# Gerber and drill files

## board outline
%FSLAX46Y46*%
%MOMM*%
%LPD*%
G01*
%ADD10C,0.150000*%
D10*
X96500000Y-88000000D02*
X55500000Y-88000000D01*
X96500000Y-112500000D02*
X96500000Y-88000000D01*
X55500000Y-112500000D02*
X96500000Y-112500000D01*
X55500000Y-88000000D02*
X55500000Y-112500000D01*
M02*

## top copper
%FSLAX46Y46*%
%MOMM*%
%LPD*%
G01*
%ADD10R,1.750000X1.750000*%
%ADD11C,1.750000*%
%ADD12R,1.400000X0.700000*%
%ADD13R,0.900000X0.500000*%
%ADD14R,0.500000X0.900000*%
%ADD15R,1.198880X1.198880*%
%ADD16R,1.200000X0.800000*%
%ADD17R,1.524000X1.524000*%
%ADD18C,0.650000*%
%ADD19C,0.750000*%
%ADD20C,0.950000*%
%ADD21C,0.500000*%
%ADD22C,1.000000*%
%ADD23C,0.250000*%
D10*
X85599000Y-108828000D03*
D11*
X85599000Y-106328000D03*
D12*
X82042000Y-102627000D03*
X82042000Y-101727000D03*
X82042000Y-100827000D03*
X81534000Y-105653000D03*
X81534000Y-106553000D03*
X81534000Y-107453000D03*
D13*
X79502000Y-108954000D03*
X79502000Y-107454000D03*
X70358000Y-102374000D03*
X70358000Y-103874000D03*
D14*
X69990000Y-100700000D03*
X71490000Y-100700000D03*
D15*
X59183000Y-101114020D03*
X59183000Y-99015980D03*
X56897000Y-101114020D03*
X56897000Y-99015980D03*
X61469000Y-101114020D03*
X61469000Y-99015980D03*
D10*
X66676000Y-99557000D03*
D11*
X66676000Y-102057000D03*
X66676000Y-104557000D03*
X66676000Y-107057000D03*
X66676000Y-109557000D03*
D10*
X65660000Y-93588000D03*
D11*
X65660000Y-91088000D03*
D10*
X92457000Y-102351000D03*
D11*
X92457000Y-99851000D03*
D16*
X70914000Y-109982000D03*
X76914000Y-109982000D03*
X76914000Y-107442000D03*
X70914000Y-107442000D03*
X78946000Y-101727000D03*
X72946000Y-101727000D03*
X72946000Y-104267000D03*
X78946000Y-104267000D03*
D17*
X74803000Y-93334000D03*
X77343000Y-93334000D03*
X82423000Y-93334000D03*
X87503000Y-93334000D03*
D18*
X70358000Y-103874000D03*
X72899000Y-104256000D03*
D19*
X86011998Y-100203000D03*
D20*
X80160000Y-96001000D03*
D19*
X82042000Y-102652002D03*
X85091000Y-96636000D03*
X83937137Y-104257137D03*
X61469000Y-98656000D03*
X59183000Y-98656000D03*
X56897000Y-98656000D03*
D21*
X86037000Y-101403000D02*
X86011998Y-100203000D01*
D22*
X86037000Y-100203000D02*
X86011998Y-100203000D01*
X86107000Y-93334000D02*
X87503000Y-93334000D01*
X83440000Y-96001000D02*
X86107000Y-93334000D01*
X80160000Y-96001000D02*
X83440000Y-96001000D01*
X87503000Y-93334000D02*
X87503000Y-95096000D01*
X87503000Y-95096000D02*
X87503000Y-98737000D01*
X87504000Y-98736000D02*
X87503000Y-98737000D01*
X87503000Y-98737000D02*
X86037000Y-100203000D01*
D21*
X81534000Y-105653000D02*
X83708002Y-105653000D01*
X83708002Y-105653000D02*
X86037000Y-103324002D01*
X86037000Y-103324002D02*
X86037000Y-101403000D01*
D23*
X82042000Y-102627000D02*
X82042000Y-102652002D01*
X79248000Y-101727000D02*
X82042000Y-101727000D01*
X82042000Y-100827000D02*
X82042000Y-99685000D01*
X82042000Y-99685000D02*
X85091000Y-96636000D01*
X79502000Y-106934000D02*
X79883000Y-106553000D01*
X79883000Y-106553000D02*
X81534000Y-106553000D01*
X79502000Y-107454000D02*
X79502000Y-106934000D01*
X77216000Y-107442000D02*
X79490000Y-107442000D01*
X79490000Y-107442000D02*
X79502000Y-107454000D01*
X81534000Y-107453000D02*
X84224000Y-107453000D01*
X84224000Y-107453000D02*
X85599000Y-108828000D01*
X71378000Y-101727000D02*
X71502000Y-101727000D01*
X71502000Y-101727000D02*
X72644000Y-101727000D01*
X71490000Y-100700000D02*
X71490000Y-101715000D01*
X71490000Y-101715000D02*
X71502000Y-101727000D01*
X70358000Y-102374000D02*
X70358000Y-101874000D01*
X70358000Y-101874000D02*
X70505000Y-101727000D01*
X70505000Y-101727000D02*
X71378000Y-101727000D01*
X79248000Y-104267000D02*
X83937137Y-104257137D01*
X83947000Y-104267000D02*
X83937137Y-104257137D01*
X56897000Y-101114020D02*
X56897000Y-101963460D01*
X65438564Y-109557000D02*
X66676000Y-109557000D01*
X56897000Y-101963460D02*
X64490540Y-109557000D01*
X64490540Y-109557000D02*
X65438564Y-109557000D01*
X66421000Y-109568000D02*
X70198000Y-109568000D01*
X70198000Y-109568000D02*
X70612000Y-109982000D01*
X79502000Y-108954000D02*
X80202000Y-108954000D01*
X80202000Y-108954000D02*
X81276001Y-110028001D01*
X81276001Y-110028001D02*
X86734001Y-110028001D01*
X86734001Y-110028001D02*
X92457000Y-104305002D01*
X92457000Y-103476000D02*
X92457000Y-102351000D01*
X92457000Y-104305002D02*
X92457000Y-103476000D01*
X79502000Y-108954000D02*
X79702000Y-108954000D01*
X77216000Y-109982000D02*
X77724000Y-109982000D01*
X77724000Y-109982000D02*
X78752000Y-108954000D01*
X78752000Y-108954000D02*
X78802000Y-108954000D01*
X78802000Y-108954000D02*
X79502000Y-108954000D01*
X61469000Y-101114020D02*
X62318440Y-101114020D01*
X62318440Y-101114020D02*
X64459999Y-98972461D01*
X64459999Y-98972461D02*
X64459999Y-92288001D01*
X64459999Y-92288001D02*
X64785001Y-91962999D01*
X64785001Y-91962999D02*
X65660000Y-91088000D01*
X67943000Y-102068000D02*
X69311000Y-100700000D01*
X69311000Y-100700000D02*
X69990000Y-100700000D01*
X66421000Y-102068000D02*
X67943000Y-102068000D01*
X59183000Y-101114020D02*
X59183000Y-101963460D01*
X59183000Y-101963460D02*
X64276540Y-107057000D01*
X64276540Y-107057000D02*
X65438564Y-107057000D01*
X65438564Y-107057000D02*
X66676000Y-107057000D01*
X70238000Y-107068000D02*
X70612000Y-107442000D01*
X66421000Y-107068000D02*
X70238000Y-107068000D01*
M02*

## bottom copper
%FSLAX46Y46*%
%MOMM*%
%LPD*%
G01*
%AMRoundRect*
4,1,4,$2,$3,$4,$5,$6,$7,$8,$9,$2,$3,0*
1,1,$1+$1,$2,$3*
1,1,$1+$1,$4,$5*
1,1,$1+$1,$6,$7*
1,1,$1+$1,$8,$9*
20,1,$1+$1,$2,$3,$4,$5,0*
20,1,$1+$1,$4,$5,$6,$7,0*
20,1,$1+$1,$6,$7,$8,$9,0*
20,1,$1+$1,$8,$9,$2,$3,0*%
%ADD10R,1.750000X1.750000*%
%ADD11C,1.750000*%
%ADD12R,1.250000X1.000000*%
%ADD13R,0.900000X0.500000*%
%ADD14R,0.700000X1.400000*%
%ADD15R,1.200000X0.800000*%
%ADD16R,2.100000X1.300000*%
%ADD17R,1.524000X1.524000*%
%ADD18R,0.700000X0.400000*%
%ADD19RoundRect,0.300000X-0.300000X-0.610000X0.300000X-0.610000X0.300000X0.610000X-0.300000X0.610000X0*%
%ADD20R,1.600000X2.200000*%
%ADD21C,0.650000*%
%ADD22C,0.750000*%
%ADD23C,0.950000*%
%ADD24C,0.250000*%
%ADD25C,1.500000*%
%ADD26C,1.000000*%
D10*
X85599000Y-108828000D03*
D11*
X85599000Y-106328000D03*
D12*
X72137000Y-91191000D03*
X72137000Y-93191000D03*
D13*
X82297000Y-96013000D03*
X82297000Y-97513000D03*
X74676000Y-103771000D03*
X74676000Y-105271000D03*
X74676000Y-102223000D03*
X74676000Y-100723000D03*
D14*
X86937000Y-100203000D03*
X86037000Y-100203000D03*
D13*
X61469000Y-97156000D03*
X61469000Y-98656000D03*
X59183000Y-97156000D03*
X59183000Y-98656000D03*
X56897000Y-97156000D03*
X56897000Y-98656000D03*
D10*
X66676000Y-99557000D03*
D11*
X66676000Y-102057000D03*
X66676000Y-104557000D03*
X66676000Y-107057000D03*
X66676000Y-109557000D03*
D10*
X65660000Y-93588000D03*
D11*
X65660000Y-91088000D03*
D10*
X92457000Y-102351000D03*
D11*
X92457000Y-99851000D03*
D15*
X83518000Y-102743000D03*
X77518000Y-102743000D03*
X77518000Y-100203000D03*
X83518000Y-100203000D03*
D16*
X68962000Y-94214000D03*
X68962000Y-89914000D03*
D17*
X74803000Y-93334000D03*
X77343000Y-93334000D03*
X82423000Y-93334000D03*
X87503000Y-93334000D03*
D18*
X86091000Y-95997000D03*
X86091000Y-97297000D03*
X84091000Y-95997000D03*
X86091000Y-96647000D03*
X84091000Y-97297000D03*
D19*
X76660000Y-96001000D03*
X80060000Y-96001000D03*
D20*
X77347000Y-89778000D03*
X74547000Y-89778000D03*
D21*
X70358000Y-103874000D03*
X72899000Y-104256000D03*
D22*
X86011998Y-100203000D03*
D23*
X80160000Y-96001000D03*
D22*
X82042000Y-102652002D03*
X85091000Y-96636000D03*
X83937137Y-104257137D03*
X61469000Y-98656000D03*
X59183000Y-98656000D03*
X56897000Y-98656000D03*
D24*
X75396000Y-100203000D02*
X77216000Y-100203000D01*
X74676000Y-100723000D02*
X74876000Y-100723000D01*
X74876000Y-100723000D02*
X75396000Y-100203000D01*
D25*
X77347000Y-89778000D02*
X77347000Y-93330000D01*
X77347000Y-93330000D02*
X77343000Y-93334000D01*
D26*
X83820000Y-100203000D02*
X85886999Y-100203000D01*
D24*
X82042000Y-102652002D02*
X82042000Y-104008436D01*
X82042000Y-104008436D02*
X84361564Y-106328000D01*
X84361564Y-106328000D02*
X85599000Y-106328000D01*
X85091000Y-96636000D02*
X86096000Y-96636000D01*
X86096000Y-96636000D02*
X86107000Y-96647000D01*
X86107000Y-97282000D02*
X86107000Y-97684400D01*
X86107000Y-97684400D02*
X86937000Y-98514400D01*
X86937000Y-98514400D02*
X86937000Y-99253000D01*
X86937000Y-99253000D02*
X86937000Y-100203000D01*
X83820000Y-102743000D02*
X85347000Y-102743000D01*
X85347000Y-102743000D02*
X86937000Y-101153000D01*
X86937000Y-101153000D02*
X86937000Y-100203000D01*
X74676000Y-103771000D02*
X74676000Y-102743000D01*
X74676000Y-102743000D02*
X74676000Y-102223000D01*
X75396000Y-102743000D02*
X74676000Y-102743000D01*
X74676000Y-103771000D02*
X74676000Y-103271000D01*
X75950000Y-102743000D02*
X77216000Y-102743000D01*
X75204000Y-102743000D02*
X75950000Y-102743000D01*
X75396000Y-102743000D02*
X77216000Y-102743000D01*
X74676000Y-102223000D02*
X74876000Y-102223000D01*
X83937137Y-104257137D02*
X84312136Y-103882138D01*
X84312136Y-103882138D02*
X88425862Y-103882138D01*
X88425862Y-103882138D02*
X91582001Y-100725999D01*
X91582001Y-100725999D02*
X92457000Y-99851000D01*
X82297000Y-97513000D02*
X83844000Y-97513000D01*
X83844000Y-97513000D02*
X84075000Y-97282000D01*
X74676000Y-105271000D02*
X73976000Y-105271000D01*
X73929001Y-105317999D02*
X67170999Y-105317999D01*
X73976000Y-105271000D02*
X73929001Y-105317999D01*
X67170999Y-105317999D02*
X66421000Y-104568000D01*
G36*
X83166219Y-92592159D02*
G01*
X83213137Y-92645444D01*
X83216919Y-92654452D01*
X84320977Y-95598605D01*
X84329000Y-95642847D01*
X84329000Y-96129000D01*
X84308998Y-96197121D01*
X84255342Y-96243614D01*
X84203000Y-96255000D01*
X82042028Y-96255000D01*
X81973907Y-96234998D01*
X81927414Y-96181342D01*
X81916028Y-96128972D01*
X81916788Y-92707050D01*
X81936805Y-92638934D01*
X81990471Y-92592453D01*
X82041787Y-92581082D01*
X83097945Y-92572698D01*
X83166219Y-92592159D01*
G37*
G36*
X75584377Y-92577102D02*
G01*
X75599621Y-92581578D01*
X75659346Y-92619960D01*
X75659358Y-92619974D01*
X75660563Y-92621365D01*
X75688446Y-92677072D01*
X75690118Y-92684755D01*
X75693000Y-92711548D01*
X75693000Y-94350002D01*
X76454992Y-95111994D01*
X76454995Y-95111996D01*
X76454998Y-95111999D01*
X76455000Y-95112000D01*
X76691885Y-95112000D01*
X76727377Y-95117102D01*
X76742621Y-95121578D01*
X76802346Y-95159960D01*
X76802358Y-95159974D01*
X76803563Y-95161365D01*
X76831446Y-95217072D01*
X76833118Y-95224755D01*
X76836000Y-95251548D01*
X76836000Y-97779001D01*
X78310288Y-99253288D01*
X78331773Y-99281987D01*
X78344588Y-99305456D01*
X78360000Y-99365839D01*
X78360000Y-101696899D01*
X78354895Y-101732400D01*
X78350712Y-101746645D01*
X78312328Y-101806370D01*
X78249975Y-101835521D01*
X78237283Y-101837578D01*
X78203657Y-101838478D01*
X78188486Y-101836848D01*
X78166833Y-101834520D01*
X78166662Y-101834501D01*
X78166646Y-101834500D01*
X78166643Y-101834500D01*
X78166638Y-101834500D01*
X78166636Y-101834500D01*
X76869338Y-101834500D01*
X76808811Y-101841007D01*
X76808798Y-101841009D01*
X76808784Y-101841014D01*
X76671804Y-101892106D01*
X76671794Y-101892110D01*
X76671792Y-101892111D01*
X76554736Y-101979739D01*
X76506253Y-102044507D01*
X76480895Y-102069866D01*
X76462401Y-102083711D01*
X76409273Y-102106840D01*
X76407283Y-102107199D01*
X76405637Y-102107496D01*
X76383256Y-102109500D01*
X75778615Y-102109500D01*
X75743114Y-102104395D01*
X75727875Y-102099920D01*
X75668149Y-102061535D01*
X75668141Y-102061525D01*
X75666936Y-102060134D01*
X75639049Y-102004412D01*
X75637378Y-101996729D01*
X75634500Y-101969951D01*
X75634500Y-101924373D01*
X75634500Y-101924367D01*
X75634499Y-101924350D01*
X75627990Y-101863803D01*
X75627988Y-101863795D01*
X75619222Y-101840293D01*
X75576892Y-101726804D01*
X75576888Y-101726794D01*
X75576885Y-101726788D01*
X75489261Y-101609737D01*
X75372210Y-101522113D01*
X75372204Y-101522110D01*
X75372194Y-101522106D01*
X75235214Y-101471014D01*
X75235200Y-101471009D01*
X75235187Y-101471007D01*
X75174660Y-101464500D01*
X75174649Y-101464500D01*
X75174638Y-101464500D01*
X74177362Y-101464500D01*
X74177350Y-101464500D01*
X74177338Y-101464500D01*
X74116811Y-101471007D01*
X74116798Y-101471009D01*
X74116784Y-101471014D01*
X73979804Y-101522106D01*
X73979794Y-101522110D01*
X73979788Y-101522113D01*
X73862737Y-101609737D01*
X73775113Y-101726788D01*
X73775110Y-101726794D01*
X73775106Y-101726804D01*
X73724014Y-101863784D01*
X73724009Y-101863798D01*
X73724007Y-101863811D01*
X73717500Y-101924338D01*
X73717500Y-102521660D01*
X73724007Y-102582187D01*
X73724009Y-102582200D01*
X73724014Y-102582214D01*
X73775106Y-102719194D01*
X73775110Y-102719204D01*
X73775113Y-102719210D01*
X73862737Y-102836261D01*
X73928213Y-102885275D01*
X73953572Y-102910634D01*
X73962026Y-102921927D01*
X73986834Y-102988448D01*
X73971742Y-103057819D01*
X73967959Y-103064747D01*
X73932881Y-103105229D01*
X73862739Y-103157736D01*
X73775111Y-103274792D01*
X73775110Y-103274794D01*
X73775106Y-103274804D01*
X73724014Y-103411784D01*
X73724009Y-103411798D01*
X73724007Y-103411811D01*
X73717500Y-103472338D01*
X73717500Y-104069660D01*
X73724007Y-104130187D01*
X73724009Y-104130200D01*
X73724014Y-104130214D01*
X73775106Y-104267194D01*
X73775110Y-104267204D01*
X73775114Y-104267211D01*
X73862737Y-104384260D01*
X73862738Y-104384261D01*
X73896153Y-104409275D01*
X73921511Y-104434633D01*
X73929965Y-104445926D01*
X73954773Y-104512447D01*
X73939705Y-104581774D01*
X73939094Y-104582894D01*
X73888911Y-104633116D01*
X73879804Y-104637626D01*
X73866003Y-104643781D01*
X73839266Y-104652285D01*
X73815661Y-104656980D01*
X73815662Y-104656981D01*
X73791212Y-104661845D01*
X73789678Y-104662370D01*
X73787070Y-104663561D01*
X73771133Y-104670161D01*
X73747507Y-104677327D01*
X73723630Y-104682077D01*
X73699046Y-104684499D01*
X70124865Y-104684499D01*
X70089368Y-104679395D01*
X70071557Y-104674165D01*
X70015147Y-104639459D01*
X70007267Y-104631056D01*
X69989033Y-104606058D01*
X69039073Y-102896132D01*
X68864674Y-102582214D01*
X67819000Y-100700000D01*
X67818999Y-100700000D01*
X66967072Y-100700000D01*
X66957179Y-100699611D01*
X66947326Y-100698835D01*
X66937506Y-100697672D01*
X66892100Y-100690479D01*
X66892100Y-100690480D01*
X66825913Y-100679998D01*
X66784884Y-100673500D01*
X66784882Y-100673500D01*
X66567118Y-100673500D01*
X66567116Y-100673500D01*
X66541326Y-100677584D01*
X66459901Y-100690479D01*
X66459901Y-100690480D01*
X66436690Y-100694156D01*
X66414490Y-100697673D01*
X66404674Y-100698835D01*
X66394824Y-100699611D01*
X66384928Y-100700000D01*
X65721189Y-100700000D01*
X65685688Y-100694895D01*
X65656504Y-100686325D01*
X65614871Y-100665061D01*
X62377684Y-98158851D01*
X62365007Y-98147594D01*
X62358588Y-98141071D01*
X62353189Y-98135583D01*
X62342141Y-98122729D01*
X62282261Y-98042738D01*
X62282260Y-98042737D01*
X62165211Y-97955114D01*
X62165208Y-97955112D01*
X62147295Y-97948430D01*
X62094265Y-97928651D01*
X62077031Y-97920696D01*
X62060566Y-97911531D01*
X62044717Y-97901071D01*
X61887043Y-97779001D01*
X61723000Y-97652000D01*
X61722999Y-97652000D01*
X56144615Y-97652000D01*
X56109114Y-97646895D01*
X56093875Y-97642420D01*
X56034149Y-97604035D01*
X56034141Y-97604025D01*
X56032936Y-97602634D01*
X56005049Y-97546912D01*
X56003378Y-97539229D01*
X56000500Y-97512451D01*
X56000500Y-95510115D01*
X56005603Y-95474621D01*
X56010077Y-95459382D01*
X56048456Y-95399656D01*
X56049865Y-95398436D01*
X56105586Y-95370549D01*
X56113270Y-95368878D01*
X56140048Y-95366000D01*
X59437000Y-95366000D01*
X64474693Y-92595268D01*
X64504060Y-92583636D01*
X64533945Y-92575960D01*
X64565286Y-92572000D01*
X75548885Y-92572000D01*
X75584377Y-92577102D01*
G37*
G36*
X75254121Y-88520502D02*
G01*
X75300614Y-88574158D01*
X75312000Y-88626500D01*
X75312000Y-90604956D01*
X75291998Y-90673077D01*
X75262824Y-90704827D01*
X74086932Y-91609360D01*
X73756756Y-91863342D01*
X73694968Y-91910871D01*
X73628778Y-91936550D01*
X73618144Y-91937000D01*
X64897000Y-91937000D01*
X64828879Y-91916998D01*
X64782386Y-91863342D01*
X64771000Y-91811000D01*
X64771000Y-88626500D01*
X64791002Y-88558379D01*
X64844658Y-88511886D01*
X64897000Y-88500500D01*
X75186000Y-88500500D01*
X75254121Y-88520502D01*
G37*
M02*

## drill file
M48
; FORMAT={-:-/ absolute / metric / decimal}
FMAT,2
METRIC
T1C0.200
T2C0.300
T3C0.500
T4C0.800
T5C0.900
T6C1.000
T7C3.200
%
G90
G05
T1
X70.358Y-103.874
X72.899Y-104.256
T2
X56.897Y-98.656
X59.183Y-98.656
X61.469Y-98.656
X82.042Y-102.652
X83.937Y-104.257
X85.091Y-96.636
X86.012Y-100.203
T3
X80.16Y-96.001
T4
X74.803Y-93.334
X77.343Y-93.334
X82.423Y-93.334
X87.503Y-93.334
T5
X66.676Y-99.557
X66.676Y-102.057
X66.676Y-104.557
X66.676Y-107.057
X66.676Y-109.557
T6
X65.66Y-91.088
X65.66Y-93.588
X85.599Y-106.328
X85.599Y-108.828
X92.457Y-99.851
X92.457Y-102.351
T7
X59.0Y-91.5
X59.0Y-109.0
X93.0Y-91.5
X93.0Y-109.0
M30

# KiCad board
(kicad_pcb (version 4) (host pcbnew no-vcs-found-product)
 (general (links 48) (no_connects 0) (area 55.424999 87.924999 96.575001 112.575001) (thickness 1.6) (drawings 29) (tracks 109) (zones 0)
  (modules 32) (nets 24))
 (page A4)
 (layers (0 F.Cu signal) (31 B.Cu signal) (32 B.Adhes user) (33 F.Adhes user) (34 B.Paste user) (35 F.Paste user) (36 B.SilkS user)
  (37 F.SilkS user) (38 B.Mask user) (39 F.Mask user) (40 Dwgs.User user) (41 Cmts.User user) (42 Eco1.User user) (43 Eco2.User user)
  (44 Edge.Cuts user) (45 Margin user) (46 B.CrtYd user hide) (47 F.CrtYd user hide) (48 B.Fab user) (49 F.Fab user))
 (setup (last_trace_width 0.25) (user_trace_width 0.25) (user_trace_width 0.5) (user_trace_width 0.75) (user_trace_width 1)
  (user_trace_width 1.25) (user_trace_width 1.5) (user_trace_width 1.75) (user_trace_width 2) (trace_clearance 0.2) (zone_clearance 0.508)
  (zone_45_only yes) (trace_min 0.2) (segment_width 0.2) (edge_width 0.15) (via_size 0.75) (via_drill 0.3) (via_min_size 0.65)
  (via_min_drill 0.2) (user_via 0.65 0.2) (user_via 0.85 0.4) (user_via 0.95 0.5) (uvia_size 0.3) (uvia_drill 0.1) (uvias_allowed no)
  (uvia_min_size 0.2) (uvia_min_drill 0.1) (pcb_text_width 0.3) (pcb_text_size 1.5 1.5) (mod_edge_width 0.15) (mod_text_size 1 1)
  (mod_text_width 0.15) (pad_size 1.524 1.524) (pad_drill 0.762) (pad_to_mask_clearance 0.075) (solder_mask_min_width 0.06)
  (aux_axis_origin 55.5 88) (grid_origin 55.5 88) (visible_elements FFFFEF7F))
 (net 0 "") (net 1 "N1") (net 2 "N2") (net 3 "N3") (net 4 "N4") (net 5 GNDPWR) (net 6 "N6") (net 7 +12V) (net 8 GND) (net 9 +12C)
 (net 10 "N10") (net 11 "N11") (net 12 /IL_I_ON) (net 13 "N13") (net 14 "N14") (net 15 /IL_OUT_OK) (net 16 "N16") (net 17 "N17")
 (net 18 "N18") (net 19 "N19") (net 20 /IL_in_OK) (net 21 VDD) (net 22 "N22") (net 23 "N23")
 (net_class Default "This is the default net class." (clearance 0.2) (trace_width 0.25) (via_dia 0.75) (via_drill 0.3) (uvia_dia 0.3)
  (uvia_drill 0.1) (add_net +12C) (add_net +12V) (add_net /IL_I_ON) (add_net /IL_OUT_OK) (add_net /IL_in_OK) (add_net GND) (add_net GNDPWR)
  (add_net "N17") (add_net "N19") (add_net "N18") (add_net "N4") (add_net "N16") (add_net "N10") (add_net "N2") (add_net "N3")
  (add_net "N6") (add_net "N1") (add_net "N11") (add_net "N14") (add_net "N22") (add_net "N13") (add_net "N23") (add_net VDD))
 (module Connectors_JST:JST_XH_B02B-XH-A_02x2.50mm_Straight (layer F.Cu) (at 85.599 108.828 90)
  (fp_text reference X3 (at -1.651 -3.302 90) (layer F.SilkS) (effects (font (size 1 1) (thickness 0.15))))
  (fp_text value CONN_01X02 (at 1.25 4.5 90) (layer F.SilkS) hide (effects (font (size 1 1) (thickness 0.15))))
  (pad 1 thru_hole rect (at 0 0 90) (size 1.75 1.75) (drill 1) (layers *.Cu *.Mask) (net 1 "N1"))
  (pad 2 thru_hole circle (at 2.5 0 90) (size 1.75 1.75) (drill 1) (layers *.Cu *.Mask) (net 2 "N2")))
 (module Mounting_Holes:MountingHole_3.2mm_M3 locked (layer F.Cu) (at 93 109)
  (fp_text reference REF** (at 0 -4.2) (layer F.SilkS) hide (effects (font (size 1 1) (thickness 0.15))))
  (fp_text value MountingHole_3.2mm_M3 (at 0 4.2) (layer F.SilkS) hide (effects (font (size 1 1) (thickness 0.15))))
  (pad 1 np_thru_hole circle (at 0 0) (size 3.2 3.2) (drill 3.2) (layers *.Cu *.Mask F.SilkS)))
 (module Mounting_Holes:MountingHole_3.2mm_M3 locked (layer F.Cu) (at 59 91.5)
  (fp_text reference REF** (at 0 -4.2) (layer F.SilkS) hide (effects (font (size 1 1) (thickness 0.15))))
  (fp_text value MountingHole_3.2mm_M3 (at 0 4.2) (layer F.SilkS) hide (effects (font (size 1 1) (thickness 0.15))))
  (pad 1 np_thru_hole circle (at 0 0) (size 3.2 3.2) (drill 3.2) (layers *.Cu *.Mask F.SilkS)))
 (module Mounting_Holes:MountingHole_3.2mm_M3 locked (layer F.Cu) (at 59 109)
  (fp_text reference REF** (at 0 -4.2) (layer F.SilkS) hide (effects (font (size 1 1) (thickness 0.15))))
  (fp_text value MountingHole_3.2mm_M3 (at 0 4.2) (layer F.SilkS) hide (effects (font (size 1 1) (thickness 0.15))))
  (pad 1 np_thru_hole circle (at 0 0) (size 3.2 3.2) (drill 3.2) (layers *.Cu *.Mask F.SilkS)))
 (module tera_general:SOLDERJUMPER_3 (layer F.Cu) (at 82.042 101.727 180)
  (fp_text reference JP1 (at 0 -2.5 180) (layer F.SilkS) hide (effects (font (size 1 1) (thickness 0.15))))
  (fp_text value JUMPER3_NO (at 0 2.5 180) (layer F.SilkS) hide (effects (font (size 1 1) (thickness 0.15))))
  (pad 1 smd rect (at 0 -0.9 180) (size 1.4 0.7) (layers F.Cu F.Paste F.Mask) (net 2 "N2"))
  (pad 2 smd rect (at 0 0 180) (size 1.4 0.7) (layers F.Cu F.Paste F.Mask) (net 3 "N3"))
  (pad 3 smd rect (at 0 0.9 180) (size 1.4 0.7) (layers F.Cu F.Paste F.Mask) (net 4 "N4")))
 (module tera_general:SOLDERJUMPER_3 (layer F.Cu) (at 81.534 106.553)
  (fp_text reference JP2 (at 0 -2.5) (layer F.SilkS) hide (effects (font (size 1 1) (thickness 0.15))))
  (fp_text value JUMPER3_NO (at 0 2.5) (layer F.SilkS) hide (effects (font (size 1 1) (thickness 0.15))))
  (pad 1 smd rect (at 0 -0.9) (size 1.4 0.7) (layers F.Cu F.Paste F.Mask) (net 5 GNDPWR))
  (pad 2 smd rect (at 0 0) (size 1.4 0.7) (layers F.Cu F.Paste F.Mask) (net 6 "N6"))
  (pad 3 smd rect (at 0 0.9) (size 1.4 0.7) (layers F.Cu F.Paste F.Mask) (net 1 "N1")))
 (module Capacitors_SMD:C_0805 (layer B.Cu) (at 72.137 92.191 270)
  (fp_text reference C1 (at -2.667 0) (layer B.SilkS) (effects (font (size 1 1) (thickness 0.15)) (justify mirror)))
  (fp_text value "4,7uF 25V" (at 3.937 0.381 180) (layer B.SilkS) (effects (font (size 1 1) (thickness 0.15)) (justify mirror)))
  (pad 1 smd rect (at -1 0 270) (size 1 1.25) (layers B.Cu B.Paste B.Mask) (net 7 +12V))
  (pad 2 smd rect (at 1 0 270) (size 1 1.25) (layers B.Cu B.Paste B.Mask) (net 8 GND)))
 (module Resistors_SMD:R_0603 (layer B.Cu) (at 82.297 96.763 270)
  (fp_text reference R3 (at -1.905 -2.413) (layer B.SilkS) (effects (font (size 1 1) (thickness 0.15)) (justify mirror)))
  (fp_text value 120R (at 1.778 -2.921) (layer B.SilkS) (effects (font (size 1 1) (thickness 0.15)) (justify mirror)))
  (pad 1 smd rect (at -0.75 0 270) (size 0.5 0.9) (layers B.Cu B.Paste B.Mask) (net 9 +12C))
  (pad 2 smd rect (at 0.75 0 270) (size 0.5 0.9) (layers B.Cu B.Paste B.Mask) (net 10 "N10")))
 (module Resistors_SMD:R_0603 (layer B.Cu) (at 74.676 104.521 270)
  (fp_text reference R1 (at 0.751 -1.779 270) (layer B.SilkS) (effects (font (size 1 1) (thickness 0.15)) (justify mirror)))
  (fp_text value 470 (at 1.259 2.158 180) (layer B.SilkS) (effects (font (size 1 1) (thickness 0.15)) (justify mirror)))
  (pad 1 smd rect (at -0.75 0 270) (size 0.5 0.9) (layers B.Cu B.Paste B.Mask) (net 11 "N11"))
  (pad 2 smd rect (at 0.75 0 270) (size 0.5 0.9) (layers B.Cu B.Paste B.Mask) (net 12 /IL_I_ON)))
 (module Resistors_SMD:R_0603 (layer B.Cu) (at 74.676 101.473 90)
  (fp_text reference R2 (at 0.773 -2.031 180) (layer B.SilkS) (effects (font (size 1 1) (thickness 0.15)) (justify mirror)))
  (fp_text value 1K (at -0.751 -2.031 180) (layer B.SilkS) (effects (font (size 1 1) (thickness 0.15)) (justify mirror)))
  (pad 1 smd rect (at -0.75 0 90) (size 0.5 0.9) (layers B.Cu B.Paste B.Mask) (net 11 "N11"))
  (pad 2 smd rect (at 0.75 0 90) (size 0.5 0.9) (layers B.Cu B.Paste B.Mask) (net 8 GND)))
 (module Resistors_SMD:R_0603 (layer F.Cu) (at 79.502 108.204 90)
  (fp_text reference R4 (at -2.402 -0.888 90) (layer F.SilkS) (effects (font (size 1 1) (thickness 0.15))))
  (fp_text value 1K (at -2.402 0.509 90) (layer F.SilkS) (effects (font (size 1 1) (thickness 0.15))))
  (pad 1 smd rect (at -0.75 0 90) (size 0.5 0.9) (layers F.Cu F.Paste F.Mask) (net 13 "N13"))
  (pad 2 smd rect (at 0.75 0 90) (size 0.5 0.9) (layers F.Cu F.Paste F.Mask) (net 6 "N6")))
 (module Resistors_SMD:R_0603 (layer F.Cu) (at 70.358 103.124 270)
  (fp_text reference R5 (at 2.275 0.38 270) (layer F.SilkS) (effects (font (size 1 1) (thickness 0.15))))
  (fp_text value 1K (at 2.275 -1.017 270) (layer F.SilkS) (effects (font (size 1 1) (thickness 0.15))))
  (pad 1 smd rect (at -0.75 0 270) (size 0.5 0.9) (layers F.Cu F.Paste F.Mask) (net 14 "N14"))
  (pad 2 smd rect (at 0.75 0 270) (size 0.5 0.9) (layers F.Cu F.Paste F.Mask) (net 8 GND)))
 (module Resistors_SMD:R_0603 (layer F.Cu) (at 70.74 100.7)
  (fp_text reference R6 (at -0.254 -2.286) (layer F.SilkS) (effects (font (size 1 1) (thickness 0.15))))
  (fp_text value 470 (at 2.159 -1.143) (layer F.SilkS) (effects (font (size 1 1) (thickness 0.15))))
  (pad 1 smd rect (at -0.75 0) (size 0.5 0.9) (layers F.Cu F.Paste F.Mask) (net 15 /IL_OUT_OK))
  (pad 2 smd rect (at 0.75 0) (size 0.5 0.9) (layers F.Cu F.Paste F.Mask) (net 14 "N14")))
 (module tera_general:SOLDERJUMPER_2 (layer B.Cu) (at 86.487 100.203 90)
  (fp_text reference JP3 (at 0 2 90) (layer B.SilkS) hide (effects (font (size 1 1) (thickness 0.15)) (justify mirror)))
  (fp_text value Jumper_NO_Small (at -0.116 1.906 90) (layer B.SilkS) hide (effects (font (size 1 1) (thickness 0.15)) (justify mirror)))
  (pad 1 smd rect (at 0 0.45 90) (size 1.4 0.7) (layers B.Cu B.Paste B.Mask) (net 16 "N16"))
  (pad 2 smd rect (at 0 -0.45 90) (size 1.4 0.7) (layers B.Cu B.Paste B.Mask) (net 5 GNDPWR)))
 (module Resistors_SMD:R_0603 (layer B.Cu) (at 61.469 97.906 270)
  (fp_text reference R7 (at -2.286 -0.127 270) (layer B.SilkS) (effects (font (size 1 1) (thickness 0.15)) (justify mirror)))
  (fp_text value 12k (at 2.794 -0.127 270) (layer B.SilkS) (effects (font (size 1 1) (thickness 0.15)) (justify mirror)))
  (pad 1 smd rect (at -0.75 0 270) (size 0.5 0.9) (layers B.Cu B.Paste B.Mask) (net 8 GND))
  (pad 2 smd rect (at 0.75 0 270) (size 0.5 0.9) (layers B.Cu B.Paste B.Mask) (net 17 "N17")))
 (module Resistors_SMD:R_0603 (layer B.Cu) (at 59.183 97.906 270)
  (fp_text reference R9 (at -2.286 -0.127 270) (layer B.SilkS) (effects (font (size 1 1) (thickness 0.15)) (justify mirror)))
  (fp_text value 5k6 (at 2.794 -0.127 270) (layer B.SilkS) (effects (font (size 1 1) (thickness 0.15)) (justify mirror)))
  (pad 1 smd rect (at -0.75 0 270) (size 0.5 0.9) (layers B.Cu B.Paste B.Mask) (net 8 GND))
  (pad 2 smd rect (at 0.75 0 270) (size 0.5 0.9) (layers B.Cu B.Paste B.Mask) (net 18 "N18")))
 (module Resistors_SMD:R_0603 (layer B.Cu) (at 56.897 97.906 270)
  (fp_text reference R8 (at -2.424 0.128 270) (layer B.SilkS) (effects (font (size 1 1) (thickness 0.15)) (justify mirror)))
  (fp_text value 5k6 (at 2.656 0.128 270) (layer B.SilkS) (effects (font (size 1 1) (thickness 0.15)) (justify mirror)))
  (pad 1 smd rect (at -0.75 0 270) (size 0.5 0.9) (layers B.Cu B.Paste B.Mask) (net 8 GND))
  (pad 2 smd rect (at 0.75 0 270) (size 0.5 0.9) (layers B.Cu B.Paste B.Mask) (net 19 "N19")))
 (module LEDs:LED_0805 (layer F.Cu) (at 59.183 100.065 270)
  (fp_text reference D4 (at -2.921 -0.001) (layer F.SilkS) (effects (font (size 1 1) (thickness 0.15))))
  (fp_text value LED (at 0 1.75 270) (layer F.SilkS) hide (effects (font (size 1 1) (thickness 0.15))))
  (pad 2 smd rect (at 1.04902 0 90) (size 1.19888 1.19888) (layers F.Cu F.Paste F.Mask) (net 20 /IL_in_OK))
  (pad 1 smd rect (at -1.04902 0 90) (size 1.19888 1.19888) (layers F.Cu F.Paste F.Mask) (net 18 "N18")))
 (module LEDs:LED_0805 (layer F.Cu) (at 56.897 100.065 270)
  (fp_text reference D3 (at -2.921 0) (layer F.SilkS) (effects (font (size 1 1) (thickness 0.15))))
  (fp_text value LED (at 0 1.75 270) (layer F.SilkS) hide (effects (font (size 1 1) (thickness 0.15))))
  (pad 2 smd rect (at 1.04902 0 90) (size 1.19888 1.19888) (layers F.Cu F.Paste F.Mask) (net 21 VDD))
  (pad 1 smd rect (at -1.04902 0 90) (size 1.19888 1.19888) (layers F.Cu F.Paste F.Mask) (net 19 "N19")))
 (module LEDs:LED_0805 (layer F.Cu) (at 61.469 100.065 270)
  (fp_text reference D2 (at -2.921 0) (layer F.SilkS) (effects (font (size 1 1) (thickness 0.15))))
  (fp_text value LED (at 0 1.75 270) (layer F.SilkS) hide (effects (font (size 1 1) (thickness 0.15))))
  (pad 2 smd rect (at 1.04902 0 90) (size 1.19888 1.19888) (layers F.Cu F.Paste F.Mask) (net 7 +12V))
  (pad 1 smd rect (at -1.04902 0 90) (size 1.19888 1.19888) (layers F.Cu F.Paste F.Mask) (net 17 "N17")))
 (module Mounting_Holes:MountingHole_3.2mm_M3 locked (layer F.Cu) (at 93 91.5)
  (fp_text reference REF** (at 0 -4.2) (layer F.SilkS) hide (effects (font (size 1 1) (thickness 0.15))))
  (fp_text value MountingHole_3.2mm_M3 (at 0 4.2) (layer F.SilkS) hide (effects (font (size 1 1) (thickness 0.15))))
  (pad 1 np_thru_hole circle (at 0 0) (size 3.2 3.2) (drill 3.2) (layers *.Cu *.Mask F.SilkS)))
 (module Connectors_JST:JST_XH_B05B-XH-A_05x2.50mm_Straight (layer F.Cu) (at 66.676 99.557 270)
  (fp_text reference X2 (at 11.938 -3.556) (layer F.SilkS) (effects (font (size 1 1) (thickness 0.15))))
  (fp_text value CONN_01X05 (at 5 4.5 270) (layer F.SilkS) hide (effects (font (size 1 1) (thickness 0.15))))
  (pad 1 thru_hole rect (at 0 0 270) (size 1.75 1.75) (drill 0.9) (layers *.Cu *.Mask) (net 8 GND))
  (pad 2 thru_hole circle (at 2.5 0 270) (size 1.75 1.75) (drill 0.9) (layers *.Cu *.Mask) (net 15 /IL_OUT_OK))
  (pad 3 thru_hole circle (at 5 0 270) (size 1.75 1.75) (drill 0.9) (layers *.Cu *.Mask) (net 12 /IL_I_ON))
  (pad 4 thru_hole circle (at 7.5 0 270) (size 1.75 1.75) (drill 0.9) (layers *.Cu *.Mask) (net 20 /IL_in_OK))
  (pad 5 thru_hole circle (at 10 0 270) (size 1.75 1.75) (drill 0.9) (layers *.Cu *.Mask) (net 21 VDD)))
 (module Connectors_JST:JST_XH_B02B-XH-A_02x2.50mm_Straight (layer F.Cu) (at 65.66 93.588 90)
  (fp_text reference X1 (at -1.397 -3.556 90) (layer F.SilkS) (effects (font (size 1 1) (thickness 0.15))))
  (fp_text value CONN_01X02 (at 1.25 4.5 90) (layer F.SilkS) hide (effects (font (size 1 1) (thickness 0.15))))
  (pad 1 thru_hole rect (at 0 0 90) (size 1.75 1.75) (drill 1) (layers *.Cu *.Mask) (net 8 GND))
  (pad 2 thru_hole circle (at 2.5 0 90) (size 1.75 1.75) (drill 1) (layers *.Cu *.Mask) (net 7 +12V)))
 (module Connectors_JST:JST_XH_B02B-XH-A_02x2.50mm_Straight (layer F.Cu) (at 92.457 102.351 90)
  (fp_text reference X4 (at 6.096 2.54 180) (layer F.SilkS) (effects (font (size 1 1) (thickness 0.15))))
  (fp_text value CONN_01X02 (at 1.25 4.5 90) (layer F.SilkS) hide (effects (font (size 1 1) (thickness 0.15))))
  (pad 1 thru_hole rect (at 0 0 90) (size 1.75 1.75) (drill 1) (layers *.Cu *.Mask) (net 13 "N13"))
  (pad 2 thru_hole circle (at 2.5 0 90) (size 1.75 1.75) (drill 1) (layers *.Cu *.Mask) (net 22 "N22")))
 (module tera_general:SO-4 (layer B.Cu) (at 80.518 101.473 90)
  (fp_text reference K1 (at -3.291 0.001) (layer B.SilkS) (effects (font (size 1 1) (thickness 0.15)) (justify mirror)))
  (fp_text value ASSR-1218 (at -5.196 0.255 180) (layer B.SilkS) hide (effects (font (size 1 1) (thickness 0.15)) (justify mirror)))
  (pad 4 smd rect (at -1.27 3 90) (size 0.8 1.2) (layers B.Cu B.Paste B.Mask) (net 16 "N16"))
  (pad 1 smd rect (at -1.27 -3 90) (size 0.8 1.2) (layers B.Cu B.Paste B.Mask) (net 11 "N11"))
  (pad 2 smd rect (at 1.27 -3 90) (size 0.8 1.2) (layers B.Cu B.Paste B.Mask) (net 8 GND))
  (pad 3 smd rect (at 1.27 3 90) (size 0.8 1.2) (layers B.Cu B.Paste B.Mask) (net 5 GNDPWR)))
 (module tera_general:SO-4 (layer F.Cu) (at 73.914 108.712 90)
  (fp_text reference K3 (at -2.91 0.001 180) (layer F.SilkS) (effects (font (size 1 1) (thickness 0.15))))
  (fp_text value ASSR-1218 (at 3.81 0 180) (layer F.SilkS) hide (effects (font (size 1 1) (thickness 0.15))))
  (pad 4 smd rect (at -1.27 -3 90) (size 0.8 1.2) (layers F.Cu F.Paste F.Mask) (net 21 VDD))
  (pad 1 smd rect (at -1.27 3 90) (size 0.8 1.2) (layers F.Cu F.Paste F.Mask) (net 13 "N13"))
  (pad 2 smd rect (at 1.27 3 90) (size 0.8 1.2) (layers F.Cu F.Paste F.Mask) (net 6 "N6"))
  (pad 3 smd rect (at 1.27 -3 90) (size 0.8 1.2) (layers F.Cu F.Paste F.Mask) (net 20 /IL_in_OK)))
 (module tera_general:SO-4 (layer F.Cu) (at 75.946 102.997 270)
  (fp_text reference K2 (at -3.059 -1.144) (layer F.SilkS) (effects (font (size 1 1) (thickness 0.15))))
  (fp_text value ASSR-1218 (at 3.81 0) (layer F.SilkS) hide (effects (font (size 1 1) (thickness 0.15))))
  (pad 4 smd rect (at -1.27 -3 270) (size 0.8 1.2) (layers F.Cu F.Paste F.Mask) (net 3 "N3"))
  (pad 1 smd rect (at -1.27 3 270) (size 0.8 1.2) (layers F.Cu F.Paste F.Mask) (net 14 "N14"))
  (pad 2 smd rect (at 1.27 3 270) (size 0.8 1.2) (layers F.Cu F.Paste F.Mask) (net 8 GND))
  (pad 3 smd rect (at 1.27 -3 270) (size 0.8 1.2) (layers F.Cu F.Paste F.Mask) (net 22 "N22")))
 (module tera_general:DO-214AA (layer B.Cu) (at 68.962 92.064 270)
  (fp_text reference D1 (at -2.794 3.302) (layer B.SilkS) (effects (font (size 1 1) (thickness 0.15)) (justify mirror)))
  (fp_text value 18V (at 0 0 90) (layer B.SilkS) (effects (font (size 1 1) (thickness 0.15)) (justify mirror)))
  (pad 2 smd rect (at 2.15 0 270) (size 1.3 2.1) (layers B.Cu B.Paste B.Mask) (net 8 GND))
  (pad 1 smd rect (at -2.15 0 270) (size 1.3 2.1) (layers B.Cu B.Paste B.Mask) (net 7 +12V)))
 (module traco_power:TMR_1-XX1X (layer F.Cu) (at 74.803 93.334)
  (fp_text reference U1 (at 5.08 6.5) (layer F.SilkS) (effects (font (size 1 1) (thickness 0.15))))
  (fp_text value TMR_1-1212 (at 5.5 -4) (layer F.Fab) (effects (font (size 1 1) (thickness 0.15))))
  (pad 1 thru_hole rect (at 0 0) (size 1.524 1.524) (drill 0.8) (layers *.Cu *.Mask) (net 8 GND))
  (pad 2 thru_hole rect (at 2.54 0) (size 1.524 1.524) (drill 0.8) (layers *.Cu *.Mask) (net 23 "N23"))
  (pad 4 thru_hole rect (at 7.62 0) (size 1.524 1.524) (drill 0.8) (layers *.Cu *.Mask) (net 9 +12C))
  (pad 6 thru_hole rect (at 12.7 0) (size 1.524 1.524) (drill 0.8) (layers *.Cu *.Mask) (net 5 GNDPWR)))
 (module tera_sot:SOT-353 (layer B.Cu) (at 85.091 96.647 180)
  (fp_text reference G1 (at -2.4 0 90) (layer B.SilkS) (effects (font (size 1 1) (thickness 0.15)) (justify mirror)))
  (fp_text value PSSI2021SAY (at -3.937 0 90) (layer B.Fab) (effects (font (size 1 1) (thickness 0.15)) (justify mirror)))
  (pad 1 smd rect (at -1 0.65 180) (size 0.7 0.4) (layers B.Cu B.Paste B.Mask))
  (pad 3 smd rect (at -1 -0.65 180) (size 0.7 0.4) (layers B.Cu B.Paste B.Mask) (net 16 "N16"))
  (pad 5 smd rect (at 1 0.65 180) (size 0.7 0.4) (layers B.Cu B.Paste B.Mask) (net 9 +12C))
  (pad 2 smd rect (at -1 0 180) (size 0.7 0.4) (layers B.Cu B.Paste B.Mask) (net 4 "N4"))
  (pad 4 smd rect (at 1 -0.65 180) (size 0.7 0.4) (layers B.Cu B.Paste B.Mask) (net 10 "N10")))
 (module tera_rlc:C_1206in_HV (layer B.Cu) (at 78.36 96.001)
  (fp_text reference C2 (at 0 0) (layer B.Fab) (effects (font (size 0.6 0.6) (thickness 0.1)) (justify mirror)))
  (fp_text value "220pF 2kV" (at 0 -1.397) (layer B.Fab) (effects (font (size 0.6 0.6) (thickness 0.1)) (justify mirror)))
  (pad 1 smd roundrect (at -1.7 0) (size 1.2 1.82) (layers B.Cu B.Paste B.Mask) (roundrect_rratio 0.25) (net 8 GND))
  (pad 2 smd roundrect (at 1.7 0) (size 1.2 1.82) (layers B.Cu B.Paste B.Mask) (roundrect_rratio 0.25) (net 5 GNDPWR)))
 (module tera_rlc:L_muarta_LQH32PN (layer B.Cu) (at 75.947 89.778 180)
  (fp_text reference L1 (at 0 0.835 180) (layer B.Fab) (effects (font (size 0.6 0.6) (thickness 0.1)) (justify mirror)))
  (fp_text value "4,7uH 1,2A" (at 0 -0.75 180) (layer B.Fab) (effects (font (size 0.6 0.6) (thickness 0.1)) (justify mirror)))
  (pad 1 smd rect (at -1.4 0 180) (size 1.6 2.2) (layers B.Cu B.Paste B.Mask) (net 23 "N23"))
  (pad 2 smd rect (at 1.4 0 180) (size 1.6 2.2) (layers B.Cu B.Paste B.Mask) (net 7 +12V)))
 (gr_line (start 96.5 88) (end 55.5 88) (layer Edge.Cuts) (width 0.15))
 (gr_line (start 96.5 112.5) (end 96.5 88) (layer Edge.Cuts) (width 0.15))
 (gr_line (start 55.5 112.5) (end 96.5 112.5) (layer Edge.Cuts) (width 0.15))
 (gr_line (start 55.5 88) (end 55.5 112.5) (layer Edge.Cuts) (width 0.15))
 (via (at 70.358 103.874) (size 0.65) (drill 0.2) (layers F.Cu B.Cu) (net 8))
 (via (at 72.899 104.256) (size 0.65) (drill 0.2) (layers F.Cu B.Cu) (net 8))
 (segment (start 75.396 100.203) (end 77.216 100.203) (width 0.25) (layer B.Cu) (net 8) (status 20))
 (segment (start 74.676 100.723) (end 74.876 100.723) (width 0.25) (layer B.Cu) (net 8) (status 30))
 (segment (start 74.876 100.723) (end 75.396 100.203) (width 0.25) (layer B.Cu) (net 8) (status 10))
 (segment (start 77.347 89.778) (end 77.347 93.33) (width 1.5) (layer B.Cu) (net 23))
 (segment (start 77.347 93.33) (end 77.343 93.334) (width 1.5) (layer B.Cu) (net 23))
 (segment (start 86.037 101.403) (end 86.011998 100.203) (width 0.5) (layer F.Cu) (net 5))
 (segment (start 86.037 100.203) (end 86.011998 100.203) (width 1) (layer F.Cu) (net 5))
 (via (at 86.011998 100.203) (size 0.75) (drill 0.3) (layers F.Cu B.Cu) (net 5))
 (segment (start 86.107 93.334) (end 87.503 93.334) (width 1) (layer F.Cu) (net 5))
 (segment (start 83.44 96.001) (end 86.107 93.334) (width 1) (layer F.Cu) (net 5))
 (segment (start 80.16 96.001) (end 83.44 96.001) (width 1) (layer F.Cu) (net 5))
 (via (at 80.16 96.001) (size 0.95) (drill 0.5) (layers F.Cu B.Cu) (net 5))
 (segment (start 87.503 93.334) (end 87.503 95.096) (width 1) (layer F.Cu) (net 5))
 (segment (start 87.503 95.096) (end 87.503 98.737) (width 1) (layer F.Cu) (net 5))
 (segment (start 87.504 98.736) (end 87.503 98.737) (width 1) (layer F.Cu) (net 5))
 (segment (start 87.503 98.737) (end 86.037 100.203) (width 1) (layer F.Cu) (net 5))
 (segment (start 81.534 105.653) (end 83.708002 105.653) (width 0.5) (layer F.Cu) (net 5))
 (segment (start 83.708002 105.653) (end 86.037 103.324002) (width 0.5) (layer F.Cu) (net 5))
 (segment (start 86.037 103.324002) (end 86.037 101.403) (width 0.5) (layer F.Cu) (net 5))
 (segment (start 83.82 100.203) (end 85.886999 100.203) (width 1) (layer B.Cu) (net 5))
 (segment (start 82.042 102.652002) (end 82.042 104.008436) (width 0.25) (layer B.Cu) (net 2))
 (segment (start 82.042 104.008436) (end 84.361564 106.328) (width 0.25) (layer B.Cu) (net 2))
 (segment (start 84.361564 106.328) (end 85.599 106.328) (width 0.25) (layer B.Cu) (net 2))
 (segment (start 82.042 102.627) (end 82.042 102.652002) (width 0.25) (layer F.Cu) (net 2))
 (via (at 82.042 102.652002) (size 0.75) (drill 0.3) (layers F.Cu B.Cu) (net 2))
 (segment (start 79.248 101.727) (end 82.042 101.727) (width 0.25) (layer F.Cu) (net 3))
 (segment (start 85.091 96.636) (end 86.096 96.636) (width 0.25) (layer B.Cu) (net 4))
 (segment (start 86.096 96.636) (end 86.107 96.647) (width 0.25) (layer B.Cu) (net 4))
 (segment (start 82.042 100.827) (end 82.042 99.685) (width 0.25) (layer F.Cu) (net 4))
 (segment (start 82.042 99.685) (end 85.091 96.636) (width 0.25) (layer F.Cu) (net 4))
 (via (at 85.091 96.636) (size 0.75) (drill 0.3) (layers F.Cu B.Cu) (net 4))
 (segment (start 79.502 106.934) (end 79.883 106.553) (width 0.25) (layer F.Cu) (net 6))
 (segment (start 79.883 106.553) (end 81.534 106.553) (width 0.25) (layer F.Cu) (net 6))
 (segment (start 79.502 107.454) (end 79.502 106.934) (width 0.25) (layer F.Cu) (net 6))
 (segment (start 77.216 107.442) (end 79.49 107.442) (width 0.25) (layer F.Cu) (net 6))
 (segment (start 79.49 107.442) (end 79.502 107.454) (width 0.25) (layer F.Cu) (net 6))
 (segment (start 81.534 107.453) (end 84.224 107.453) (width 0.25) (layer F.Cu) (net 1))
 (segment (start 84.224 107.453) (end 85.599 108.828) (width 0.25) (layer F.Cu) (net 1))
 (segment (start 86.107 97.282) (end 86.107 97.6844) (width 0.25) (layer B.Cu) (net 16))
 (segment (start 86.107 97.6844) (end 86.937 98.5144) (width 0.25) (layer B.Cu) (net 16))
 (segment (start 86.937 98.5144) (end 86.937 99.253) (width 0.25) (layer B.Cu) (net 16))
 (segment (start 86.937 99.253) (end 86.937 100.203) (width 0.25) (layer B.Cu) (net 16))
 (segment (start 83.82 102.743) (end 85.347 102.743) (width 0.25) (layer B.Cu) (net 16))
 (segment (start 85.347 102.743) (end 86.937 101.153) (width 0.25) (layer B.Cu) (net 16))
 (segment (start 86.937 101.153) (end 86.937 100.203) (width 0.25) (layer B.Cu) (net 16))
 (segment (start 74.676 103.771) (end 74.676 102.743) (width 0.25) (layer B.Cu) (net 11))
 (segment (start 74.676 102.743) (end 74.676 102.223) (width 0.25) (layer B.Cu) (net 11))
 (segment (start 75.396 102.743) (end 74.676 102.743) (width 0.25) (layer B.Cu) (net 11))
 (segment (start 74.676 103.771) (end 74.676 103.271) (width 0.25) (layer B.Cu) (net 11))
 (segment (start 75.95 102.743) (end 77.216 102.743) (width 0.25) (layer B.Cu) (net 11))
 (segment (start 75.204 102.743) (end 75.95 102.743) (width 0.25) (layer B.Cu) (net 11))
 (segment (start 75.396 102.743) (end 77.216 102.743) (width 0.25) (layer B.Cu) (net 11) (status 20))
 (segment (start 74.676 102.223) (end 74.876 102.223) (width 0.25) (layer B.Cu) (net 11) (status 30))
 (segment (start 71.378 101.727) (end 71.502 101.727) (width 0.25) (layer F.Cu) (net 14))
 (segment (start 71.502 101.727) (end 72.644 101.727) (width 0.25) (layer F.Cu) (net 14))
 (segment (start 71.49 100.7) (end 71.49 101.715) (width 0.25) (layer F.Cu) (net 14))
 (segment (start 71.49 101.715) (end 71.502 101.727) (width 0.25) (layer F.Cu) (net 14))
 (segment (start 70.358 102.374) (end 70.358 101.874) (width 0.25) (layer F.Cu) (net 14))
 (segment (start 70.358 101.874) (end 70.505 101.727) (width 0.25) (layer F.Cu) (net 14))
 (segment (start 70.505 101.727) (end 71.378 101.727) (width 0.25) (layer F.Cu) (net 14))
 (segment (start 83.937137 104.257137) (end 84.312136 103.882138) (width 0.25) (layer B.Cu) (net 22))
 (segment (start 84.312136 103.882138) (end 88.425862 103.882138) (width 0.25) (layer B.Cu) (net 22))
 (segment (start 88.425862 103.882138) (end 91.582001 100.725999) (width 0.25) (layer B.Cu) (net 22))
 (segment (start 91.582001 100.725999) (end 92.457 99.851) (width 0.25) (layer B.Cu) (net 22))
 (segment (start 79.248 104.267) (end 83.937137 104.257137) (width 0.25) (layer F.Cu) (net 22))
 (segment (start 83.947 104.267) (end 83.937137 104.257137) (width 0.25) (layer F.Cu) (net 22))
 (via (at 83.937137 104.257137) (size 0.75) (drill 0.3) (layers F.Cu B.Cu) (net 22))
 (segment (start 56.897 101.11402) (end 56.897 101.96346) (width 0.25) (layer F.Cu) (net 21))
 (segment (start 65.438564 109.557) (end 66.676 109.557) (width 0.25) (layer F.Cu) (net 21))
 (segment (start 56.897 101.96346) (end 64.49054 109.557) (width 0.25) (layer F.Cu) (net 21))
 (segment (start 64.49054 109.557) (end 65.438564 109.557) (width 0.25) (layer F.Cu) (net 21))
 (segment (start 66.421 109.568) (end 70.198 109.568) (width 0.25) (layer F.Cu) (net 21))
 (segment (start 70.198 109.568) (end 70.612 109.982) (width 0.25) (layer F.Cu) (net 21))
 (segment (start 79.502 108.954) (end 80.202 108.954) (width 0.25) (layer F.Cu) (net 13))
 (segment (start 80.202 108.954) (end 81.276001 110.028001) (width 0.25) (layer F.Cu) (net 13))
 (segment (start 81.276001 110.028001) (end 86.734001 110.028001) (width 0.25) (layer F.Cu) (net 13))
 (segment (start 86.734001 110.028001) (end 92.457 104.305002) (width 0.25) (layer F.Cu) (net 13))
 (segment (start 92.457 103.476) (end 92.457 102.351) (width 0.25) (layer F.Cu) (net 13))
 (segment (start 92.457 104.305002) (end 92.457 103.476) (width 0.25) (layer F.Cu) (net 13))
 (segment (start 79.502 108.954) (end 79.702 108.954) (width 0.25) (layer F.Cu) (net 13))
 (segment (start 77.216 109.982) (end 77.724 109.982) (width 0.25) (layer F.Cu) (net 13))
 (segment (start 77.724 109.982) (end 78.752 108.954) (width 0.25) (layer F.Cu) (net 13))
 (segment (start 78.752 108.954) (end 78.802 108.954) (width 0.25) (layer F.Cu) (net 13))
 (segment (start 78.802 108.954) (end 79.502 108.954) (width 0.25) (layer F.Cu) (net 13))
 (segment (start 61.469 101.11402) (end 62.31844 101.11402) (width 0.25) (layer F.Cu) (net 7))
 (segment (start 62.31844 101.11402) (end 64.459999 98.972461) (width 0.25) (layer F.Cu) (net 7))
 (segment (start 64.459999 98.972461) (end 64.459999 92.288001) (width 0.25) (layer F.Cu) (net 7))
 (segment (start 64.459999 92.288001) (end 64.785001 91.962999) (width 0.25) (layer F.Cu) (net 7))
 (segment (start 64.785001 91.962999) (end 65.66 91.088) (width 0.25) (layer F.Cu) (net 7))
 (segment (start 82.297 97.513) (end 83.844 97.513) (width 0.25) (layer B.Cu) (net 10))
 (segment (start 83.844 97.513) (end 84.075 97.282) (width 0.25) (layer B.Cu) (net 10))
 (segment (start 74.676 105.271) (end 73.976 105.271) (width 0.25) (layer B.Cu) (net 12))
 (segment (start 73.929001 105.317999) (end 67.170999 105.317999) (width 0.25) (layer B.Cu) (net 12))
 (segment (start 73.976 105.271) (end 73.929001 105.317999) (width 0.25) (layer B.Cu) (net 12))
 (segment (start 67.170999 105.317999) (end 66.421 104.568) (width 0.25) (layer B.Cu) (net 12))
 (segment (start 67.943 102.068) (end 69.311 100.7) (width 0.25) (layer F.Cu) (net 15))
 (segment (start 69.311 100.7) (end 69.99 100.7) (width 0.25) (layer F.Cu) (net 15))
 (segment (start 66.421 102.068) (end 67.943 102.068) (width 0.25) (layer F.Cu) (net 15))
 (via (at 61.469 98.656) (size 0.75) (drill 0.3) (layers F.Cu B.Cu) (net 17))
 (via (at 59.183 98.656) (size 0.75) (drill 0.3) (layers F.Cu B.Cu) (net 18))
 (via (at 56.897 98.656) (size 0.75) (drill 0.3) (layers F.Cu B.Cu) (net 19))
 (segment (start 59.183 101.11402) (end 59.183 101.96346) (width 0.25) (layer F.Cu) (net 20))
 (segment (start 59.183 101.96346) (end 64.27654 107.057) (width 0.25) (layer F.Cu) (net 20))
 (segment (start 64.27654 107.057) (end 65.438564 107.057) (width 0.25) (layer F.Cu) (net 20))
 (segment (start 65.438564 107.057) (end 66.676 107.057) (width 0.25) (layer F.Cu) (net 20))
 (segment (start 70.238 107.068) (end 70.612 107.442) (width 0.25) (layer F.Cu) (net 20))
 (segment (start 66.421 107.068) (end 70.238 107.068) (width 0.25) (layer F.Cu) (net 20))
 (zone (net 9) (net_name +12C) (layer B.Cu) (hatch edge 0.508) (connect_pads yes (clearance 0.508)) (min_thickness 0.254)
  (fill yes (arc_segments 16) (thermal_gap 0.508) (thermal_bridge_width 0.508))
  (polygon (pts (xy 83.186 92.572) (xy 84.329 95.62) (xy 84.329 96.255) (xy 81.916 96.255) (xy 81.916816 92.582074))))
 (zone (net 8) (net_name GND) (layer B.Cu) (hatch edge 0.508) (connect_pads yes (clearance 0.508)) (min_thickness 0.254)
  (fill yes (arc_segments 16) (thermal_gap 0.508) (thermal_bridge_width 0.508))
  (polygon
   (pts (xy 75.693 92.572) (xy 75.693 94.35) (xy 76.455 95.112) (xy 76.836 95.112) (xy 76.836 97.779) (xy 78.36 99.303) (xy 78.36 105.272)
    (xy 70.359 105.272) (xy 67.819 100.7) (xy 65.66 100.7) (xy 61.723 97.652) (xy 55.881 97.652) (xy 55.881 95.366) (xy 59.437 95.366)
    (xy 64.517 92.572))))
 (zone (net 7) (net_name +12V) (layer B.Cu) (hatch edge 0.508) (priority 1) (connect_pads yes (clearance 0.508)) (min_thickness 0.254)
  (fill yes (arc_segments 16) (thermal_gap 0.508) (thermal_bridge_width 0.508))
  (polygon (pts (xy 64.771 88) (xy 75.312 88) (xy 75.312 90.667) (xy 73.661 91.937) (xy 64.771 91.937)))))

